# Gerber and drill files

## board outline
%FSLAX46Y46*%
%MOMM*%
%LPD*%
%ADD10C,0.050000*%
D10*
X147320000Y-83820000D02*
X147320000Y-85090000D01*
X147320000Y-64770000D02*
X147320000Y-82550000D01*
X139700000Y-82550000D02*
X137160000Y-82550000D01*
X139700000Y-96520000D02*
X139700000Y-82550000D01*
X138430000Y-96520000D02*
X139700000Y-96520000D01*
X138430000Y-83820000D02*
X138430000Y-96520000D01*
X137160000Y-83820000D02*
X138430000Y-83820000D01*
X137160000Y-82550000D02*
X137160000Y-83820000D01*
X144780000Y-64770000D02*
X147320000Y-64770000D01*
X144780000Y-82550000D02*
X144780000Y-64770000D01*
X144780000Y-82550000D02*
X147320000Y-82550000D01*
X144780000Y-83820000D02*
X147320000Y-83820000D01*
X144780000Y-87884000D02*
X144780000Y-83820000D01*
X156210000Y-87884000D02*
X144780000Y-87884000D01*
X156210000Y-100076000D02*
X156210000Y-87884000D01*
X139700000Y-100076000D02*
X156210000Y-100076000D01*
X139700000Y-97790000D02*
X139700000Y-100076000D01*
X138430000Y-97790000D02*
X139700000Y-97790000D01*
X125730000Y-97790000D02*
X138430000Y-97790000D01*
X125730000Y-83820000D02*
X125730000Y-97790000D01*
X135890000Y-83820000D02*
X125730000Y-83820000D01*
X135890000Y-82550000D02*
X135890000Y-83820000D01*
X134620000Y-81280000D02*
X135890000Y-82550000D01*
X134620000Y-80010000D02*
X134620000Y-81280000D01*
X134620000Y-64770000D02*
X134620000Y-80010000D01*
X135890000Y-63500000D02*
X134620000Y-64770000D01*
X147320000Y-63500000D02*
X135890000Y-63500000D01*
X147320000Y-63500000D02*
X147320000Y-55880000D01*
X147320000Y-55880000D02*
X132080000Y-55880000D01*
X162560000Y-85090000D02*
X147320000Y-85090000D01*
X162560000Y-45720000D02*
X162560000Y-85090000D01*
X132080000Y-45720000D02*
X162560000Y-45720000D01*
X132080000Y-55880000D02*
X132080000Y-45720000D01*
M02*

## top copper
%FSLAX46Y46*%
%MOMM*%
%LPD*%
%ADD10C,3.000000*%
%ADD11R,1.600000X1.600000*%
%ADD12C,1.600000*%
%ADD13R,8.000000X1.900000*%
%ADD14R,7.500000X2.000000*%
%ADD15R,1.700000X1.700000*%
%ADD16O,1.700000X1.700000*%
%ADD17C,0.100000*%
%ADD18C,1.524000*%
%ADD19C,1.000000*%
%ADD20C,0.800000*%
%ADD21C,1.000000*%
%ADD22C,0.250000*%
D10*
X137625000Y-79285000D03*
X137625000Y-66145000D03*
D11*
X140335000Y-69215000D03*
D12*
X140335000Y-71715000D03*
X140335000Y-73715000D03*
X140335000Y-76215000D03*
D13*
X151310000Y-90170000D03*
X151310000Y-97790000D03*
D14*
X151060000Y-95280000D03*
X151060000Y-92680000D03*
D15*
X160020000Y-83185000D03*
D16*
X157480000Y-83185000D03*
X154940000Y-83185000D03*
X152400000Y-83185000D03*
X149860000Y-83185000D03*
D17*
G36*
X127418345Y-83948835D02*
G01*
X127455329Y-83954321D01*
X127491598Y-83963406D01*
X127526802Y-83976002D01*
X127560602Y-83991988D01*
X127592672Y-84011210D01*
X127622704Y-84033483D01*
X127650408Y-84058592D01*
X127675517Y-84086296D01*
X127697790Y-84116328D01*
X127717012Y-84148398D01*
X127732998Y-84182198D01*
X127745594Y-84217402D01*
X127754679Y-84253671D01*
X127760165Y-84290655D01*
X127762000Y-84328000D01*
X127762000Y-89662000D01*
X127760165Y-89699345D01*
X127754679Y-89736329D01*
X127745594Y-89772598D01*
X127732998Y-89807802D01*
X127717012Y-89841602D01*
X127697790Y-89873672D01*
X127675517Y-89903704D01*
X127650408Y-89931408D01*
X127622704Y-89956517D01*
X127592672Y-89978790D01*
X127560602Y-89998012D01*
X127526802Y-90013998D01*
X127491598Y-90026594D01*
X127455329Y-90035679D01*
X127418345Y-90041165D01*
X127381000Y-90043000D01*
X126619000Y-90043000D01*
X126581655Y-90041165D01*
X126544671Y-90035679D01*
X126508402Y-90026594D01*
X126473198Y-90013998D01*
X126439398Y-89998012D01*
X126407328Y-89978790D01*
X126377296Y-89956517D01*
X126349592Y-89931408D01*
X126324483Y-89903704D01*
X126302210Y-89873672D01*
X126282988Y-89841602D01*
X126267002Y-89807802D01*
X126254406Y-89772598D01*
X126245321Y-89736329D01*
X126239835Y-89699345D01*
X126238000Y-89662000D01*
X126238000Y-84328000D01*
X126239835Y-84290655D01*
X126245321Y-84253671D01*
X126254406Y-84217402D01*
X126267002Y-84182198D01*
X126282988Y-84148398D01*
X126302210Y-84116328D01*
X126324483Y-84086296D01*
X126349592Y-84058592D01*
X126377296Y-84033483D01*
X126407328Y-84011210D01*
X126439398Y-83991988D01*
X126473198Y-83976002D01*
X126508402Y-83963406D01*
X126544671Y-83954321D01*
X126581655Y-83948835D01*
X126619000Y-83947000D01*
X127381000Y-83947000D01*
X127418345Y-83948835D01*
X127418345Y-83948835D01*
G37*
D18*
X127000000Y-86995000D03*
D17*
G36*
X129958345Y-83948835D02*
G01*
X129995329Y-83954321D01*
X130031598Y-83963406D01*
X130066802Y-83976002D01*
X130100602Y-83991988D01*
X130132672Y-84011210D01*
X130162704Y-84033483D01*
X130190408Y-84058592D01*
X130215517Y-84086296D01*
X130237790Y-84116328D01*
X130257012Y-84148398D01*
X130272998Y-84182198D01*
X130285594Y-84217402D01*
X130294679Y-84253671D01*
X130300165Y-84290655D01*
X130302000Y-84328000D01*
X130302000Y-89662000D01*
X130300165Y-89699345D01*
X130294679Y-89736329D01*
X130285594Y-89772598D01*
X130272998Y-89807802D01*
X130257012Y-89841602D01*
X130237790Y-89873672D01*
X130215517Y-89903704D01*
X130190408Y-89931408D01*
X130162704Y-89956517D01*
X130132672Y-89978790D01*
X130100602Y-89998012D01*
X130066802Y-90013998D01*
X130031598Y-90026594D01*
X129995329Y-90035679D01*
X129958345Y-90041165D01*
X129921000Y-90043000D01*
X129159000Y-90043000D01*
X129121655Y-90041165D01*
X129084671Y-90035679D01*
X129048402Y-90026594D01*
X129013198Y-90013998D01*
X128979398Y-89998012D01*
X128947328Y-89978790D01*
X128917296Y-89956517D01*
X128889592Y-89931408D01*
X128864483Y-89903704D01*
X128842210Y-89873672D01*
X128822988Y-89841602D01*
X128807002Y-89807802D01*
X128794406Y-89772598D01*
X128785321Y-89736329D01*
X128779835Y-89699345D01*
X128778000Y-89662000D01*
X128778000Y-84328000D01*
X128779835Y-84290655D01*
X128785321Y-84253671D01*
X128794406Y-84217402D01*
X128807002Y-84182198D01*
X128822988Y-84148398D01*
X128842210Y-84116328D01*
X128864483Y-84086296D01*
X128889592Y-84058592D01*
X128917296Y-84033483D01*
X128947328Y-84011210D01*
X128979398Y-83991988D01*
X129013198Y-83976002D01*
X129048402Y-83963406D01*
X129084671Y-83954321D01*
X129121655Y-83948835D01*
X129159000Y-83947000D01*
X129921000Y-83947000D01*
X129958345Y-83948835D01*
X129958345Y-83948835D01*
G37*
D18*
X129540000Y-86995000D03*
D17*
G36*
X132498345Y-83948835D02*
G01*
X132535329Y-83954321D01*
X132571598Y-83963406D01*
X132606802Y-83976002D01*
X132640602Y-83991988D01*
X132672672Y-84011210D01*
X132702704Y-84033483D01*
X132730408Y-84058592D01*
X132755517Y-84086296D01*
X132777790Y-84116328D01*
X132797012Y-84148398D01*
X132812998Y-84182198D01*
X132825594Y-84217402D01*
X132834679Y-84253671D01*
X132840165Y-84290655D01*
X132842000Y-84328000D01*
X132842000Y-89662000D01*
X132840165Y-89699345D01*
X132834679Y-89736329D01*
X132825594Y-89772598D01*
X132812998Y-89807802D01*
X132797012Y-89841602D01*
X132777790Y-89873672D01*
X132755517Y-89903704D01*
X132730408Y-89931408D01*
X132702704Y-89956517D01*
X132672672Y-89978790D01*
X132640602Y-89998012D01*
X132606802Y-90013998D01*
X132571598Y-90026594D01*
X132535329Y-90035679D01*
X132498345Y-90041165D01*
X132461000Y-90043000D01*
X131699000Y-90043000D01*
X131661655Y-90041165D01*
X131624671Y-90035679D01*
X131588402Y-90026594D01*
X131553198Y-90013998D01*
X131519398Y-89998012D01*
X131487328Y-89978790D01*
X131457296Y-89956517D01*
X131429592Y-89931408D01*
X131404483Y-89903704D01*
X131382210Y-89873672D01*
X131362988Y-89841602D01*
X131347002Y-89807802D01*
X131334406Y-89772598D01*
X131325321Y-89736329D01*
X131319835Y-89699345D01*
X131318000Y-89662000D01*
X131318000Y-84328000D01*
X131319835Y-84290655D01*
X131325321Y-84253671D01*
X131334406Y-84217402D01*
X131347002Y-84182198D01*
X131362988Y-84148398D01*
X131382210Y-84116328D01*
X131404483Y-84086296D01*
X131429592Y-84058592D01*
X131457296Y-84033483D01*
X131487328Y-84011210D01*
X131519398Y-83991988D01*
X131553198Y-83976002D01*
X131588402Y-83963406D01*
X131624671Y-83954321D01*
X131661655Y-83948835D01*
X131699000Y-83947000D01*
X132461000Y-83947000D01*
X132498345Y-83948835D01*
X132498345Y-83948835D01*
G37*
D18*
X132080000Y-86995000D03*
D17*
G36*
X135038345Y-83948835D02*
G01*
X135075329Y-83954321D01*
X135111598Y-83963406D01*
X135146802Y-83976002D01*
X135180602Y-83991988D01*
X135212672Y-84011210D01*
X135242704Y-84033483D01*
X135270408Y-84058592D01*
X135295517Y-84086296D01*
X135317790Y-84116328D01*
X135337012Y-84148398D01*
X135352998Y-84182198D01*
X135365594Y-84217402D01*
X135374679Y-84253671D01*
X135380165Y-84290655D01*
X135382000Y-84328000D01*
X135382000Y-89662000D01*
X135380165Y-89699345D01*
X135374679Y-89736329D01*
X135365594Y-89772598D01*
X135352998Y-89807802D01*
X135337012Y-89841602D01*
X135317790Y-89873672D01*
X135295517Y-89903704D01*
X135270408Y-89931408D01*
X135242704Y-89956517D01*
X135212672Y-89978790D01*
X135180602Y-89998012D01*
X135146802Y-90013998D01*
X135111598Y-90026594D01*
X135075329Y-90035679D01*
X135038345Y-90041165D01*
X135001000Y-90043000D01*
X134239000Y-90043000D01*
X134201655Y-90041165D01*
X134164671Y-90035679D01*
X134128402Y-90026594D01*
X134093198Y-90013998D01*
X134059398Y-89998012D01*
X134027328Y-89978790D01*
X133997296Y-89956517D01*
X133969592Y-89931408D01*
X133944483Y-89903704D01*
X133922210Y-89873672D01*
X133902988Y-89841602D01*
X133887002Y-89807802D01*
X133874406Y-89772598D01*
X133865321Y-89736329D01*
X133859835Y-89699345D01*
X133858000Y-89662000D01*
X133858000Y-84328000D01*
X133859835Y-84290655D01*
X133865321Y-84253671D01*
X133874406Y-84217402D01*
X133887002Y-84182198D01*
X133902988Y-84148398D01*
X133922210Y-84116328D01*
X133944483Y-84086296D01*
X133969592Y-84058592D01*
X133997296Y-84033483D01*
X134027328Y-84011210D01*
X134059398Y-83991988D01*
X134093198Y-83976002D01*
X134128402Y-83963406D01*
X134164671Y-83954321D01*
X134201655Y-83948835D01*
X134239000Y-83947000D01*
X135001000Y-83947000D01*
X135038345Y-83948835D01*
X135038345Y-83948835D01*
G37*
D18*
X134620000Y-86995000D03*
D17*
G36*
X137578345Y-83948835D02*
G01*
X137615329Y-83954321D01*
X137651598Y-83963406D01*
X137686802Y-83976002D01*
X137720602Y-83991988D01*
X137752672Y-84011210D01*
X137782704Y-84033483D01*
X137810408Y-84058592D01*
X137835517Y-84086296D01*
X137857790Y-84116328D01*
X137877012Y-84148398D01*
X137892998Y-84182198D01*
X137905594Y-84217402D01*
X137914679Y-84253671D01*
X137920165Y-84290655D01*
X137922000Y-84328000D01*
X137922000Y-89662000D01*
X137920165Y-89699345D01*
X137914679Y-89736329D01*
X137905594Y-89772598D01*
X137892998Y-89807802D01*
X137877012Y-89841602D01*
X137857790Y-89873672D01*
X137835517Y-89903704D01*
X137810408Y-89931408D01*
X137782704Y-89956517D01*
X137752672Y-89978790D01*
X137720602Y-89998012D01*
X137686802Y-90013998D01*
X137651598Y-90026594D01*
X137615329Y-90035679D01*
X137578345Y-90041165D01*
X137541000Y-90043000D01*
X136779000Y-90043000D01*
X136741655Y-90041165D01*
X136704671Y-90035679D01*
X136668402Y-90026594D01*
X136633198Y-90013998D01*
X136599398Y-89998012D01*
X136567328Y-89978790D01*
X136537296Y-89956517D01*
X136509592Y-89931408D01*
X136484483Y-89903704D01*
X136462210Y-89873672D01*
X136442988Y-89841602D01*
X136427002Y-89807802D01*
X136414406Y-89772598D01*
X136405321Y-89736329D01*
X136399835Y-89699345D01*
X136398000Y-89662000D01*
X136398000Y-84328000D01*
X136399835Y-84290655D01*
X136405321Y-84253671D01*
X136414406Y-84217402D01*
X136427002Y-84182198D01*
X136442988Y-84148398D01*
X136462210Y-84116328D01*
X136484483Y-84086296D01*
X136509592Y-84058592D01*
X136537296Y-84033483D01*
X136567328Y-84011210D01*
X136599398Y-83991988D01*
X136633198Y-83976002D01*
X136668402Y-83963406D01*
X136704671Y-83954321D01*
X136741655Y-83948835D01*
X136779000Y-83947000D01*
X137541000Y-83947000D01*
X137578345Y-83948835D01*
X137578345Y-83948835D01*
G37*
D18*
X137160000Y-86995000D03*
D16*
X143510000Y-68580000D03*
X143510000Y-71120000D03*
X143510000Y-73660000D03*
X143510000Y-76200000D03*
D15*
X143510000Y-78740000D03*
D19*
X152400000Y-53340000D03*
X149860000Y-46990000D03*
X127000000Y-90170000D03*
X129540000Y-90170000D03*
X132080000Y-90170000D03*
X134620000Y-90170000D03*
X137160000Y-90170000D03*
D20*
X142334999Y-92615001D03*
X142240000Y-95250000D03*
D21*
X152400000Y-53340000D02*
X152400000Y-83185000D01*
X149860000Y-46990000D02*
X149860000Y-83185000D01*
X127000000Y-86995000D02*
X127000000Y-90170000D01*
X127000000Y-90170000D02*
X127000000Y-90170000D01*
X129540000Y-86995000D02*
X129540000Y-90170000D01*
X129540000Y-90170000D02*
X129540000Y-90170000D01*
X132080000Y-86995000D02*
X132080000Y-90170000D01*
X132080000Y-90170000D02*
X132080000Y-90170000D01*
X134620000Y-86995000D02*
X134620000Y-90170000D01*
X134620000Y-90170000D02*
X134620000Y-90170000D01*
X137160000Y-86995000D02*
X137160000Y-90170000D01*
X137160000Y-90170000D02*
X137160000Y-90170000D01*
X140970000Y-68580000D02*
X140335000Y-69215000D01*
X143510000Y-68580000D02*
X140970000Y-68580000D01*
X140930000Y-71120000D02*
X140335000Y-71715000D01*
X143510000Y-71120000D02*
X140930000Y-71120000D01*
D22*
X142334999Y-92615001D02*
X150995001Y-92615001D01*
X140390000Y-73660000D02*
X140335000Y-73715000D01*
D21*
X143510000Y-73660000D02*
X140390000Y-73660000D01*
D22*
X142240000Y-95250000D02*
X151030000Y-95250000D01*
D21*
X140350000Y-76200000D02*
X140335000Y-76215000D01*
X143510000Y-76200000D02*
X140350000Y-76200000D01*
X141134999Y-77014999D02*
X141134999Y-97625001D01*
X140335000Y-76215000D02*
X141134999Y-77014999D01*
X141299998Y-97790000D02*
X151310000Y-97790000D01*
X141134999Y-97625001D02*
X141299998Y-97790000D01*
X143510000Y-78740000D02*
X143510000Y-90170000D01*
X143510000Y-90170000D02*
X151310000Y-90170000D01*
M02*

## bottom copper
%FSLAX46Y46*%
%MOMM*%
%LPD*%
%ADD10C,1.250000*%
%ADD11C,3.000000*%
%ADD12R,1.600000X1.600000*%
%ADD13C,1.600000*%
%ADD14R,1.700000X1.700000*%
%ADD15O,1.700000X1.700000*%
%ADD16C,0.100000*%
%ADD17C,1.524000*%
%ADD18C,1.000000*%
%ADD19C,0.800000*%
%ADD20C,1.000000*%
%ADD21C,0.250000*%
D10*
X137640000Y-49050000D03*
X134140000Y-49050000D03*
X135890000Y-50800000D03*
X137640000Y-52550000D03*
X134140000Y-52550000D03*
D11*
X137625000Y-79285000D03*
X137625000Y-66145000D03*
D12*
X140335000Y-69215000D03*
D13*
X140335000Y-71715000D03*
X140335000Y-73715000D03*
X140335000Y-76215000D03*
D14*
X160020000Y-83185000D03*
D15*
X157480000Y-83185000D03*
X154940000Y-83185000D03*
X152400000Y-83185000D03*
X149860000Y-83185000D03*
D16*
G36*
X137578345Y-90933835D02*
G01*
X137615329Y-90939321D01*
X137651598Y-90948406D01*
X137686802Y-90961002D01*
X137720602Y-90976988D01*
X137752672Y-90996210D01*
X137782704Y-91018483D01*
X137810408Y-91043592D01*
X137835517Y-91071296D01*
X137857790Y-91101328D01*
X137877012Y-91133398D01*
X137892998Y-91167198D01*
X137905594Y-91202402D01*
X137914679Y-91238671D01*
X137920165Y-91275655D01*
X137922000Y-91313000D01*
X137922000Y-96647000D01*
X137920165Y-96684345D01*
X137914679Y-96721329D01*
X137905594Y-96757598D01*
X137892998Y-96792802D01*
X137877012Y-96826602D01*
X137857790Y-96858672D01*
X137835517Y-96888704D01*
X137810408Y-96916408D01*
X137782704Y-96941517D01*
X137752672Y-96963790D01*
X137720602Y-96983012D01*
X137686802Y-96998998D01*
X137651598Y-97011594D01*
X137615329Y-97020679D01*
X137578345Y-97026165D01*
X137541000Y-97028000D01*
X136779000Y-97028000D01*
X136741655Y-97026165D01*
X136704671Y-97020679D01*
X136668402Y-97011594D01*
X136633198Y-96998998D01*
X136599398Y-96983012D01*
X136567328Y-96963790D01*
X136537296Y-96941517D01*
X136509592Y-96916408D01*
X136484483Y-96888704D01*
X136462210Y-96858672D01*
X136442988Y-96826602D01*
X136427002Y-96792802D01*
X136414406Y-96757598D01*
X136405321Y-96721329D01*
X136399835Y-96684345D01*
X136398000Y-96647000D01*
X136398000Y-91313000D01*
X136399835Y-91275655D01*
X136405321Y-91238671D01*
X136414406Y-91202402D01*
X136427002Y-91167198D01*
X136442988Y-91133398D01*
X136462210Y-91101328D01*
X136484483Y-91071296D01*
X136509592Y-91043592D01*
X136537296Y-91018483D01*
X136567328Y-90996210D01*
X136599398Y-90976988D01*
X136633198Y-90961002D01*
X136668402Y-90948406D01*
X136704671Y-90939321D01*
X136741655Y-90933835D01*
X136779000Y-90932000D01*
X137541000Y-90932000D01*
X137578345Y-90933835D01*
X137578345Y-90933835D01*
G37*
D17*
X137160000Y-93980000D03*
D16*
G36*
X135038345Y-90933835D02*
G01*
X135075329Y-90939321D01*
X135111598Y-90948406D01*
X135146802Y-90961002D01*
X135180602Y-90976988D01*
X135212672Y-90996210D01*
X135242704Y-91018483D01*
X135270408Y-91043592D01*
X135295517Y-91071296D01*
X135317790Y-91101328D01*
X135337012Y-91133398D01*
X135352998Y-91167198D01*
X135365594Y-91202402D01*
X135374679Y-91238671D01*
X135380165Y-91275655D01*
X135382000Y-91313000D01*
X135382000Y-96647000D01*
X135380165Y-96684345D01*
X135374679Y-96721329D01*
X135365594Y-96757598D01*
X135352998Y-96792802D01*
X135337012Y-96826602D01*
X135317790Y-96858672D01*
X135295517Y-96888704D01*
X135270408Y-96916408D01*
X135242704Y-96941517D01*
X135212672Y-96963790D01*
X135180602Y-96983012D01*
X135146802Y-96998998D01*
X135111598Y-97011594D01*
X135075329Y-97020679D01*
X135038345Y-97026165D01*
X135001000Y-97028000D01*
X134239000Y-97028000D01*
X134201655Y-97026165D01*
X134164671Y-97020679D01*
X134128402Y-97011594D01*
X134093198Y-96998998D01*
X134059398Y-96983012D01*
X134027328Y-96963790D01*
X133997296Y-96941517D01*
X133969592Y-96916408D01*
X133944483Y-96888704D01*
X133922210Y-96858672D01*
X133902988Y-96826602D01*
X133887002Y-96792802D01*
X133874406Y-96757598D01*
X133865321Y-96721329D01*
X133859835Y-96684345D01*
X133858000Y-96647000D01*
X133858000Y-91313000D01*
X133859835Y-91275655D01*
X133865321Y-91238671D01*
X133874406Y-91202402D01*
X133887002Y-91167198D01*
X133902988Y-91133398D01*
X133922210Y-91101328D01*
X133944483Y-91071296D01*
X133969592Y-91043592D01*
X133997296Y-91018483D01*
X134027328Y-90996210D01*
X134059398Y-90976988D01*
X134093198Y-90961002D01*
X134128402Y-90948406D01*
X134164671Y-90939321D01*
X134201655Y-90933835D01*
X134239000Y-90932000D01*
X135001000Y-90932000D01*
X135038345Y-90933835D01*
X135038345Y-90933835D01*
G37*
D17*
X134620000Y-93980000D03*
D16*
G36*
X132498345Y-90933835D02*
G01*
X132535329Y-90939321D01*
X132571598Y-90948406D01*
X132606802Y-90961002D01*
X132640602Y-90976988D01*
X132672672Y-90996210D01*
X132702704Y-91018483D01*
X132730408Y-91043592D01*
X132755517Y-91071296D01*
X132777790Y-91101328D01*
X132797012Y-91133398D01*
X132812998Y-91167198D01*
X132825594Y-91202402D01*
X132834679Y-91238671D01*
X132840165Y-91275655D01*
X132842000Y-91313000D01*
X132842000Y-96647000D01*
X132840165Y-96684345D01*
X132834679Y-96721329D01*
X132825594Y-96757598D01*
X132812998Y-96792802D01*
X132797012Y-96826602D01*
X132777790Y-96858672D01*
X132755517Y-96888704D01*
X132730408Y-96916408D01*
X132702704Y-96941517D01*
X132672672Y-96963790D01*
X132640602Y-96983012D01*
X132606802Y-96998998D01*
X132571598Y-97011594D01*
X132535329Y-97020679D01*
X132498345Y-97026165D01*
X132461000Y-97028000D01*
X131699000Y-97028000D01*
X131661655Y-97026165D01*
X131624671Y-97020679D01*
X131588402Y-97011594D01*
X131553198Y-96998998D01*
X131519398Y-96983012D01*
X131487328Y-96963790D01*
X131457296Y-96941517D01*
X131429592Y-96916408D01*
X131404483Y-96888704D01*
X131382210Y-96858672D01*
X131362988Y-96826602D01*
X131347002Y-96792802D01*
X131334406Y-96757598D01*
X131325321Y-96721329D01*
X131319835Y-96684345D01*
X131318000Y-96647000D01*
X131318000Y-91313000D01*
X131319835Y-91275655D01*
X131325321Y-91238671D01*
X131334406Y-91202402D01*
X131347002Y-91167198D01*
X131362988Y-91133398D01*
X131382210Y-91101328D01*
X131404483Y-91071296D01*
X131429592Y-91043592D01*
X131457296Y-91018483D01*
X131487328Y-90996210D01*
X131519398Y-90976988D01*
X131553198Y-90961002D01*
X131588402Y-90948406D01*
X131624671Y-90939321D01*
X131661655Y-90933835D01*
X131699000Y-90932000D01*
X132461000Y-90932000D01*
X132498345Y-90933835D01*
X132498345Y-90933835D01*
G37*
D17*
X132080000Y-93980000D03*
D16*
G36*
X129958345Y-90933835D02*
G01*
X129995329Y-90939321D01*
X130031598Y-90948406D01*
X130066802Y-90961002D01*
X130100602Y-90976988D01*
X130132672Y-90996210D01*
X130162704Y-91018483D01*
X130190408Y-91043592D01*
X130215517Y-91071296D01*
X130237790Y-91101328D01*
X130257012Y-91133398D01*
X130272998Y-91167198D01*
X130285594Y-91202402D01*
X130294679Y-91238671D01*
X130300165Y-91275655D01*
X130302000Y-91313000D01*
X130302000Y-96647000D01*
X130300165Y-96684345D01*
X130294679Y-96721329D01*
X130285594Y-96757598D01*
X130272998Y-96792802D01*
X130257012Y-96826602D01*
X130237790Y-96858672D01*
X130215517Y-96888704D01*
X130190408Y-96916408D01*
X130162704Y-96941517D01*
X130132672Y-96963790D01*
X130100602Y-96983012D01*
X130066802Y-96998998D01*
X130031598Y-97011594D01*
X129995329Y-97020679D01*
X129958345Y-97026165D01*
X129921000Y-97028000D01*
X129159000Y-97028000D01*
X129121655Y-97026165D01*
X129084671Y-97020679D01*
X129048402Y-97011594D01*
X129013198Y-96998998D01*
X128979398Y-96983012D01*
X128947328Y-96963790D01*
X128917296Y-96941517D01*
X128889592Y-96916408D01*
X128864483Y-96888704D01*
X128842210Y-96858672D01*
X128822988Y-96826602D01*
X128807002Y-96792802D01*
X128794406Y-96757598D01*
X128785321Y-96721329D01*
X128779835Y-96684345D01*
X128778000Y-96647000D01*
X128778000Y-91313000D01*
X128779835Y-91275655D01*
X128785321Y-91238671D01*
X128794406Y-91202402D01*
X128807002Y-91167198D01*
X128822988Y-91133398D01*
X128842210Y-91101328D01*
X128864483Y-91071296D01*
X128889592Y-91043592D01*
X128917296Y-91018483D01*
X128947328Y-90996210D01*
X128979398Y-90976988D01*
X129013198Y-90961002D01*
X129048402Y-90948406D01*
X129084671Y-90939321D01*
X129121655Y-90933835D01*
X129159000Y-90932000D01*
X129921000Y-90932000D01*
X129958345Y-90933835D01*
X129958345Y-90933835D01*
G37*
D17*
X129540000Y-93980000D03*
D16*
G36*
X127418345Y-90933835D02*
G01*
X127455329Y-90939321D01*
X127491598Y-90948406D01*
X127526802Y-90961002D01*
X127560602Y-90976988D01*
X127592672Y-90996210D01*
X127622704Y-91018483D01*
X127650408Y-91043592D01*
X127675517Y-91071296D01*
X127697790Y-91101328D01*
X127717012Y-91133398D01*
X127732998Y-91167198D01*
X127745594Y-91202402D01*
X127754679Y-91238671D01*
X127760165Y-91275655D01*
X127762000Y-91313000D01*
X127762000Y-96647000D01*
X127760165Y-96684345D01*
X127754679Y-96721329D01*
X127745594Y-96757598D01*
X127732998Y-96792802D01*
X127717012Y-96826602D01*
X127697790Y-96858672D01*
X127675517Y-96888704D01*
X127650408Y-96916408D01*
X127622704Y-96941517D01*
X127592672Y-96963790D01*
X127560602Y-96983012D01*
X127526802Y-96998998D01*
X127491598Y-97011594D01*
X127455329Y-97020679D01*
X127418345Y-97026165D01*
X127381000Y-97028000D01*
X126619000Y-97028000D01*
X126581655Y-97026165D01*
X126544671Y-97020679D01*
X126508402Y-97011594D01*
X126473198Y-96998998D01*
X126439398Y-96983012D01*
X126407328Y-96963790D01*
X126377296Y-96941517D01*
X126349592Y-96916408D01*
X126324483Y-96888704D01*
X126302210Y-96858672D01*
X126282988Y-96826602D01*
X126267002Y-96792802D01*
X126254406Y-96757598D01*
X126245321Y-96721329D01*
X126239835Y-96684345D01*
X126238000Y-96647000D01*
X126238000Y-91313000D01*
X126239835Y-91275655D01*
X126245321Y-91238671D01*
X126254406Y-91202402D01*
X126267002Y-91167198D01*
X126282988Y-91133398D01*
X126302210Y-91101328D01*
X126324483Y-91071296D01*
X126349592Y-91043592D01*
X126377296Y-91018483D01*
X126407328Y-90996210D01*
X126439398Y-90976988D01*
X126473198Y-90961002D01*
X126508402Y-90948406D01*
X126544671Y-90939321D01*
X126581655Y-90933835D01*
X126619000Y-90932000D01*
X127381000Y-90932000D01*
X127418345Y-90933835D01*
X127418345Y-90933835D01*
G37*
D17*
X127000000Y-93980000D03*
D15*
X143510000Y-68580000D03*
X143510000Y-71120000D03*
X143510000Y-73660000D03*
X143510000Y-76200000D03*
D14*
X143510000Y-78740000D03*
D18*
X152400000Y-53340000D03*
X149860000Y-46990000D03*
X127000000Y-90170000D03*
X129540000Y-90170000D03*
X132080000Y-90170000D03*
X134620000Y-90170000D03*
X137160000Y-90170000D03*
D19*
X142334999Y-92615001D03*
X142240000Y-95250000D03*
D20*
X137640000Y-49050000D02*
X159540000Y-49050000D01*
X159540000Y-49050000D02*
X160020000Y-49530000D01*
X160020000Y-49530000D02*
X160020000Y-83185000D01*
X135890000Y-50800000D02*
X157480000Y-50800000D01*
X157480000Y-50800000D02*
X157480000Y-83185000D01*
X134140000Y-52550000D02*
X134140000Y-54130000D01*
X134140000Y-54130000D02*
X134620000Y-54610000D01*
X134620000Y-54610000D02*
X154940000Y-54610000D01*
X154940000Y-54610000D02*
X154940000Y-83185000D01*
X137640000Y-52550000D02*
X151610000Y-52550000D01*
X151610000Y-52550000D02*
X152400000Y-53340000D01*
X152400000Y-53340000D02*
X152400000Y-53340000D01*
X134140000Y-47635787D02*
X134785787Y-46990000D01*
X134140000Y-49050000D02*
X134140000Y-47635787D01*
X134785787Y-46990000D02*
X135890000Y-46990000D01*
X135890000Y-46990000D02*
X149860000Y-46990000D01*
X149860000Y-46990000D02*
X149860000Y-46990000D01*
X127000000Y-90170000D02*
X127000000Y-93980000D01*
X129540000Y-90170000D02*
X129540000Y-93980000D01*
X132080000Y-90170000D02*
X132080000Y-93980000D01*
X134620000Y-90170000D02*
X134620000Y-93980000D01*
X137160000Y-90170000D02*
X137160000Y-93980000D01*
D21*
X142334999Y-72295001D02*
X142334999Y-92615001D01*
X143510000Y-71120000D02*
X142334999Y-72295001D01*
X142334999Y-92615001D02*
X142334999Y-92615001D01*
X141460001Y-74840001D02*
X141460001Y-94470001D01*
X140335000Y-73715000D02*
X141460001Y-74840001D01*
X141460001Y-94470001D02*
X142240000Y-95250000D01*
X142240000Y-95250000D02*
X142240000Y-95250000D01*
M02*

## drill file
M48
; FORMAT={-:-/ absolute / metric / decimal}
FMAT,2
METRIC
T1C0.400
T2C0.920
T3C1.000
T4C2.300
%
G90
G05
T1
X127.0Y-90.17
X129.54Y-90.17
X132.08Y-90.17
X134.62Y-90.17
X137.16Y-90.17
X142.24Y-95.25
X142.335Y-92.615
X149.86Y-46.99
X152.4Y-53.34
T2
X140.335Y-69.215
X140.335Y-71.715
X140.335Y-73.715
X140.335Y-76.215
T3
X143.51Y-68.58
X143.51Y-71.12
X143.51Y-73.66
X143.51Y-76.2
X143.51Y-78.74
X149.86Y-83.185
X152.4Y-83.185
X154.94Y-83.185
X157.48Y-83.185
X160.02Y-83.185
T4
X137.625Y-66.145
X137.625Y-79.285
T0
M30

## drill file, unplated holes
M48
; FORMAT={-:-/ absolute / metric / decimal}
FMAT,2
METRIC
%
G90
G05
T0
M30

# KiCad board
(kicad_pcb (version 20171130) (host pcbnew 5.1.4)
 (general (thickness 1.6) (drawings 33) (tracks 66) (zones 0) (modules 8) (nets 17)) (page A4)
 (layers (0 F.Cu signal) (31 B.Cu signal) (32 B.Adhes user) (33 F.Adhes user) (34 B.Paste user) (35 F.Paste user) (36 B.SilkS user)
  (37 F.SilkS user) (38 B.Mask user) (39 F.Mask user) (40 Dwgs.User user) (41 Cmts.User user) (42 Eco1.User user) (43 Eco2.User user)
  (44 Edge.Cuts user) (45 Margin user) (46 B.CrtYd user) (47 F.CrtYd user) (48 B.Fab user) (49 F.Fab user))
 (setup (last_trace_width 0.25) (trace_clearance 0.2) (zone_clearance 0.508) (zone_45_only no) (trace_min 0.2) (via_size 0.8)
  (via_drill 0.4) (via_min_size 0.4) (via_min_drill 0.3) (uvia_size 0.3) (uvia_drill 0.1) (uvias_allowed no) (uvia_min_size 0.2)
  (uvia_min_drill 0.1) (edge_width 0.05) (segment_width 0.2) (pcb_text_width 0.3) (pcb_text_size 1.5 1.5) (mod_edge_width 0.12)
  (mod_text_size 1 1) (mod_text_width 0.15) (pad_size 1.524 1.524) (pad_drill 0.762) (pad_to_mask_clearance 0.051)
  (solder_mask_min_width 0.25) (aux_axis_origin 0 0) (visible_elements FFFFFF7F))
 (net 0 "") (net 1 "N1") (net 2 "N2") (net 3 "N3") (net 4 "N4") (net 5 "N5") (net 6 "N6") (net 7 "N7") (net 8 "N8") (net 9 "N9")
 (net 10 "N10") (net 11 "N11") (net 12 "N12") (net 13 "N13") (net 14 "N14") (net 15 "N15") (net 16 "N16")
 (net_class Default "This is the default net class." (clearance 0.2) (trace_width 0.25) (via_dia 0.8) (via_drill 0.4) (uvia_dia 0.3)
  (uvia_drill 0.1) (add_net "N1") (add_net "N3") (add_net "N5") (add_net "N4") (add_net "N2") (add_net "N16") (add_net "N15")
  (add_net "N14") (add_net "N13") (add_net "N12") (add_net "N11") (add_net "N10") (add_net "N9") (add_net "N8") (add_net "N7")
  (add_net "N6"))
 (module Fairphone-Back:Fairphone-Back (layer F.Cu) (at 135.89 50.8)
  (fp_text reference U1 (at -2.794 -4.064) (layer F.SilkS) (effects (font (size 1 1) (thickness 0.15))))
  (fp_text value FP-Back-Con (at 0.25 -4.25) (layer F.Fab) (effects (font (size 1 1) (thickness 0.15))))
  (pad 2 connect circle (at 1.75 -1.75) (size 1.25 1.25) (layers B.Cu B.Mask) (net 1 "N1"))
  (pad 1 connect circle (at -1.75 -1.75) (size 1.25 1.25) (layers B.Cu B.Mask) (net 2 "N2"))
  (pad 3 connect circle (at 0 0) (size 1.25 1.25) (layers B.Cu B.Mask) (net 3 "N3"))
  (pad 5 connect circle (at 1.75 1.75) (size 1.25 1.25) (layers B.Cu B.Mask) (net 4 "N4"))
  (pad 4 connect circle (at -1.75 1.75) (size 1.25 1.25) (layers B.Cu B.Mask) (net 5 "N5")))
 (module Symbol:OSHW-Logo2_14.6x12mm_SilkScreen (layer F.Cu) (at 154.94 51.816)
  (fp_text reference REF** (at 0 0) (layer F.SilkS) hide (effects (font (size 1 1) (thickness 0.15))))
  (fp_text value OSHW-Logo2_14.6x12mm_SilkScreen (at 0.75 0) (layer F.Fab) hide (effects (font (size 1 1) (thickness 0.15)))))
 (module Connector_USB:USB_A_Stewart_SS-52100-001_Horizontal (layer F.Cu) (at 140.335 69.215 270)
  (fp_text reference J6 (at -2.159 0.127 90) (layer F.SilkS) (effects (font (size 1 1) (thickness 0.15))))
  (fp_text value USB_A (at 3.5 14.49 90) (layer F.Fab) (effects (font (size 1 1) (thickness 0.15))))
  (pad 5 thru_hole circle (at 10.07 2.71 270) (size 3 3) (drill 2.3) (layers *.Cu *.Mask) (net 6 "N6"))
  (pad 5 thru_hole circle (at -3.07 2.71 270) (size 3 3) (drill 2.3) (layers *.Cu *.Mask) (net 6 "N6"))
  (pad 1 thru_hole rect (at 0 0 270) (size 1.6 1.6) (drill 0.92) (layers *.Cu *.Mask) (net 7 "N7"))
  (pad 2 thru_hole circle (at 2.5 0 270) (size 1.6 1.6) (drill 0.92) (layers *.Cu *.Mask) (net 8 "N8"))
  (pad 3 thru_hole circle (at 4.5 0 270) (size 1.6 1.6) (drill 0.92) (layers *.Cu *.Mask) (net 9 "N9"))
  (pad 4 thru_hole circle (at 7 0 270) (size 1.6 1.6) (drill 0.92) (layers *.Cu *.Mask) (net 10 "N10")))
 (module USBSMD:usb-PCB (layer F.Cu) (at 156.21 93.98 90)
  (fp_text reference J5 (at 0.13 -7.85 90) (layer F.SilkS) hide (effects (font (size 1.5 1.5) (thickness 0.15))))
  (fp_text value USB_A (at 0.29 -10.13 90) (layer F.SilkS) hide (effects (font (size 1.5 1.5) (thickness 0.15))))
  (pad 1 connect rect (at 3.81 -4.9 90) (size 1.9 8) (layers F.Cu F.Mask) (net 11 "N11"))
  (pad 4 connect rect (at -3.81 -4.9 90) (size 1.9 8) (layers F.Cu F.Mask) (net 10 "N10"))
  (pad 3 connect rect (at -1.3 -5.15 90) (size 2 7.5) (layers F.Cu F.Mask) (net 9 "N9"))
  (pad 2 connect rect (at 1.3 -5.15 90) (size 2 7.5) (layers F.Cu F.Mask) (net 8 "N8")))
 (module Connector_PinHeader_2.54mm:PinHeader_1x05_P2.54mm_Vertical (layer F.Cu) (at 160.02 83.185 270)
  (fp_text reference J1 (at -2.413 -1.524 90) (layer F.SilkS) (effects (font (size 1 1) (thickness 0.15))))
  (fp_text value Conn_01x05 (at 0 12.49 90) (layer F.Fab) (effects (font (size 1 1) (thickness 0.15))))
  (pad 1 thru_hole rect (at 0 0 270) (size 1.7 1.7) (drill 1) (layers *.Cu *.Mask) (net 1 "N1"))
  (pad 2 thru_hole oval (at 0 2.54 270) (size 1.7 1.7) (drill 1) (layers *.Cu *.Mask) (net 3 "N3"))
  (pad 3 thru_hole oval (at 0 5.08 270) (size 1.7 1.7) (drill 1) (layers *.Cu *.Mask) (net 5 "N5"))
  (pad 4 thru_hole oval (at 0 7.62 270) (size 1.7 1.7) (drill 1) (layers *.Cu *.Mask) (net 4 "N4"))
  (pad 5 thru_hole oval (at 0 10.16 270) (size 1.7 1.7) (drill 1) (layers *.Cu *.Mask) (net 2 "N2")))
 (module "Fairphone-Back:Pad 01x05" (layer B.Cu) (at 132.08 93.98)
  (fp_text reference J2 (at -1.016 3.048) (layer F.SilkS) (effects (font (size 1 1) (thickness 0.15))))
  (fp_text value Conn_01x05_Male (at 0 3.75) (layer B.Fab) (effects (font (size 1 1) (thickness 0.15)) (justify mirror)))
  (pad 5 smd roundrect (at 5.08 0) (size 1.524 6.096) (layers B.Cu B.Paste B.Mask) (roundrect_rratio 0.25) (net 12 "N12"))
  (pad 4 smd roundrect (at 2.54 0) (size 1.524 6.096) (layers B.Cu B.Paste B.Mask) (roundrect_rratio 0.25) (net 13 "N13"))
  (pad 3 smd roundrect (at 0 0) (size 1.524 6.096) (layers B.Cu B.Paste B.Mask) (roundrect_rratio 0.25) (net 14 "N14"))
  (pad 2 smd roundrect (at -2.54 0) (size 1.524 6.096) (layers B.Cu B.Paste B.Mask) (roundrect_rratio 0.25) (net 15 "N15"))
  (pad 1 smd roundrect (at -5.08 0) (size 1.524 6.096) (layers B.Cu B.Paste B.Mask) (roundrect_rratio 0.25) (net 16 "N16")))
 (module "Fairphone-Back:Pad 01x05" (layer F.Cu) (at 132.08 86.995)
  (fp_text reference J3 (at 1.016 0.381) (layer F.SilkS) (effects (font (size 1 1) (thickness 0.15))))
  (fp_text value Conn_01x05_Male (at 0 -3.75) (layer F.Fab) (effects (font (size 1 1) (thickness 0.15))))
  (pad 1 smd roundrect (at -5.08 0) (size 1.524 6.096) (layers F.Cu F.Paste F.Mask) (roundrect_rratio 0.25) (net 16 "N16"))
  (pad 2 smd roundrect (at -2.54 0) (size 1.524 6.096) (layers F.Cu F.Paste F.Mask) (roundrect_rratio 0.25) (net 15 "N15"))
  (pad 3 smd roundrect (at 0 0) (size 1.524 6.096) (layers F.Cu F.Paste F.Mask) (roundrect_rratio 0.25) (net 14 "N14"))
  (pad 4 smd roundrect (at 2.54 0) (size 1.524 6.096) (layers F.Cu F.Paste F.Mask) (roundrect_rratio 0.25) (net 13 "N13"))
  (pad 5 smd roundrect (at 5.08 0) (size 1.524 6.096) (layers F.Cu F.Paste F.Mask) (roundrect_rratio 0.25) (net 12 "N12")))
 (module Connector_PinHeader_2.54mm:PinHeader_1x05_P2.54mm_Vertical (layer F.Cu) (at 143.51 78.74 180)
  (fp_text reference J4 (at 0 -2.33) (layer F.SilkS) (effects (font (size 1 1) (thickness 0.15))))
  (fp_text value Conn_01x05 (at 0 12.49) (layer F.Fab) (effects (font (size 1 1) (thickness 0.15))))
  (pad 5 thru_hole oval (at 0 10.16 180) (size 1.7 1.7) (drill 1) (layers *.Cu *.Mask) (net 7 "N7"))
  (pad 4 thru_hole oval (at 0 7.62 180) (size 1.7 1.7) (drill 1) (layers *.Cu *.Mask) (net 8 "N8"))
  (pad 3 thru_hole oval (at 0 5.08 180) (size 1.7 1.7) (drill 1) (layers *.Cu *.Mask) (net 9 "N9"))
  (pad 2 thru_hole oval (at 0 2.54 180) (size 1.7 1.7) (drill 1) (layers *.Cu *.Mask) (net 10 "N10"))
  (pad 1 thru_hole rect (at 0 0 180) (size 1.7 1.7) (drill 1) (layers *.Cu *.Mask) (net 11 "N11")))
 (gr_line (start 147.32 83.82) (end 147.32 85.09) (layer Edge.Cuts) (width 0.05))
 (gr_line (start 147.32 64.77) (end 147.32 82.55) (layer Edge.Cuts) (width 0.05))
 (gr_line (start 139.7 82.55) (end 137.16 82.55) (layer Edge.Cuts) (width 0.05))
 (gr_line (start 139.7 96.52) (end 139.7 82.55) (layer Edge.Cuts) (width 0.05))
 (gr_line (start 138.43 96.52) (end 139.7 96.52) (layer Edge.Cuts) (width 0.05))
 (gr_line (start 138.43 83.82) (end 138.43 96.52) (layer Edge.Cuts) (width 0.05))
 (gr_line (start 137.16 83.82) (end 138.43 83.82) (layer Edge.Cuts) (width 0.05))
 (gr_line (start 137.16 82.55) (end 137.16 83.82) (layer Edge.Cuts) (width 0.05))
 (gr_line (start 144.78 64.77) (end 147.32 64.77) (layer Edge.Cuts) (width 0.05))
 (gr_line (start 144.78 82.55) (end 144.78 64.77) (layer Edge.Cuts) (width 0.05))
 (gr_line (start 144.78 82.55) (end 147.32 82.55) (layer Edge.Cuts) (width 0.05))
 (gr_line (start 144.78 83.82) (end 147.32 83.82) (layer Edge.Cuts) (width 0.05))
 (gr_line (start 144.78 87.884) (end 144.78 83.82) (layer Edge.Cuts) (width 0.05))
 (gr_line (start 156.21 87.884) (end 144.78 87.884) (layer Edge.Cuts) (width 0.05))
 (gr_line (start 156.21 100.076) (end 156.21 87.884) (layer Edge.Cuts) (width 0.05))
 (gr_line (start 139.7 100.076) (end 156.21 100.076) (layer Edge.Cuts) (width 0.05))
 (gr_line (start 139.7 97.79) (end 139.7 100.076) (layer Edge.Cuts) (width 0.05))
 (gr_line (start 138.43 97.79) (end 139.7 97.79) (layer Edge.Cuts) (width 0.05))
 (gr_line (start 125.73 97.79) (end 138.43 97.79) (layer Edge.Cuts) (width 0.05))
 (gr_line (start 125.73 83.82) (end 125.73 97.79) (layer Edge.Cuts) (width 0.05))
 (gr_line (start 135.89 83.82) (end 125.73 83.82) (layer Edge.Cuts) (width 0.05))
 (gr_line (start 135.89 82.55) (end 135.89 83.82) (layer Edge.Cuts) (width 0.05))
 (gr_line (start 134.62 81.28) (end 135.89 82.55) (layer Edge.Cuts) (width 0.05))
 (gr_line (start 134.62 80.01) (end 134.62 81.28) (layer Edge.Cuts) (width 0.05))
 (gr_line (start 134.62 64.77) (end 134.62 80.01) (layer Edge.Cuts) (width 0.05))
 (gr_line (start 135.89 63.5) (end 134.62 64.77) (layer Edge.Cuts) (width 0.05))
 (gr_line (start 147.32 63.5) (end 135.89 63.5) (layer Edge.Cuts) (width 0.05))
 (gr_line (start 147.32 63.5) (end 147.32 55.88) (layer Edge.Cuts) (width 0.05))
 (gr_line (start 147.32 55.88) (end 132.08 55.88) (layer Edge.Cuts) (width 0.05))
 (gr_line (start 162.56 85.09) (end 147.32 85.09) (layer Edge.Cuts) (width 0.05))
 (gr_line (start 162.56 45.72) (end 162.56 85.09) (layer Edge.Cuts) (width 0.05))
 (gr_line (start 132.08 45.72) (end 162.56 45.72) (layer Edge.Cuts) (width 0.05))
 (gr_line (start 132.08 55.88) (end 132.08 45.72) (layer Edge.Cuts) (width 0.05))
 (segment (start 137.64 49.05) (end 159.54 49.05) (width 1) (layer B.Cu) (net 1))
 (segment (start 159.54 49.05) (end 160.02 49.53) (width 1) (layer B.Cu) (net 1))
 (segment (start 160.02 49.53) (end 160.02 83.185) (width 1) (layer B.Cu) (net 1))
 (segment (start 135.89 50.8) (end 157.48 50.8) (width 1) (layer B.Cu) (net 3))
 (segment (start 157.48 50.8) (end 157.48 83.185) (width 1) (layer B.Cu) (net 3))
 (segment (start 134.14 52.55) (end 134.14 54.13) (width 1) (layer B.Cu) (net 5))
 (segment (start 134.14 54.13) (end 134.62 54.61) (width 1) (layer B.Cu) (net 5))
 (segment (start 134.62 54.61) (end 154.94 54.61) (width 1) (layer B.Cu) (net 5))
 (segment (start 154.94 54.61) (end 154.94 83.185) (width 1) (layer B.Cu) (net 5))
 (segment (start 137.64 52.55) (end 151.61 52.55) (width 1) (layer B.Cu) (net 4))
 (segment (start 151.61 52.55) (end 152.4 53.34) (width 1) (layer B.Cu) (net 4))
 (segment (start 152.4 53.34) (end 152.4 53.34) (width 1) (layer B.Cu) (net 4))
 (via (at 152.4 53.34) (size 1) (drill 0.4) (layers F.Cu B.Cu) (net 4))
 (segment (start 152.4 53.34) (end 152.4 83.185) (width 1) (layer F.Cu) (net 4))
 (segment (start 134.14 47.635787) (end 134.785787 46.99) (width 1) (layer B.Cu) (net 2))
 (segment (start 134.14 49.05) (end 134.14 47.635787) (width 1) (layer B.Cu) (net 2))
 (segment (start 134.785787 46.99) (end 135.89 46.99) (width 1) (layer B.Cu) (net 2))
 (segment (start 135.89 46.99) (end 149.86 46.99) (width 1) (layer B.Cu) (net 2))
 (segment (start 149.86 46.99) (end 149.86 46.99) (width 1) (layer B.Cu) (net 2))
 (via (at 149.86 46.99) (size 1) (drill 0.4) (layers F.Cu B.Cu) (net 2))
 (segment (start 149.86 46.99) (end 149.86 83.185) (width 1) (layer F.Cu) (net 2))
 (segment (start 127 86.995) (end 127 90.17) (width 1) (layer F.Cu) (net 16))
 (segment (start 127 90.17) (end 127 90.17) (width 1) (layer F.Cu) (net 16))
 (via (at 127 90.17) (size 1) (drill 0.4) (layers F.Cu B.Cu) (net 16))
 (segment (start 127 90.17) (end 127 93.98) (width 1) (layer B.Cu) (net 16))
 (segment (start 129.54 86.995) (end 129.54 90.17) (width 1) (layer F.Cu) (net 15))
 (segment (start 129.54 90.17) (end 129.54 90.17) (width 1) (layer F.Cu) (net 15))
 (via (at 129.54 90.17) (size 1) (drill 0.4) (layers F.Cu B.Cu) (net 15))
 (segment (start 129.54 90.17) (end 129.54 93.98) (width 1) (layer B.Cu) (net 15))
 (segment (start 132.08 86.995) (end 132.08 90.17) (width 1) (layer F.Cu) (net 14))
 (segment (start 132.08 90.17) (end 132.08 90.17) (width 1) (layer F.Cu) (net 14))
 (via (at 132.08 90.17) (size 1) (drill 0.4) (layers F.Cu B.Cu) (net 14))
 (segment (start 132.08 90.17) (end 132.08 93.98) (width 1) (layer B.Cu) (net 14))
 (segment (start 134.62 86.995) (end 134.62 90.17) (width 1) (layer F.Cu) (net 13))
 (segment (start 134.62 90.17) (end 134.62 90.17) (width 1) (layer F.Cu) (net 13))
 (via (at 134.62 90.17) (size 1) (drill 0.4) (layers F.Cu B.Cu) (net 13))
 (segment (start 134.62 90.17) (end 134.62 93.98) (width 1) (layer B.Cu) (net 13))
 (segment (start 137.16 86.995) (end 137.16 90.17) (width 1) (layer F.Cu) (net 12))
 (segment (start 137.16 90.17) (end 137.16 90.17) (width 1) (layer F.Cu) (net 12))
 (via (at 137.16 90.17) (size 1) (drill 0.4) (layers F.Cu B.Cu) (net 12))
 (segment (start 137.16 90.17) (end 137.16 93.98) (width 1) (layer B.Cu) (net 12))
 (segment (start 140.97 68.58) (end 140.335 69.215) (width 1) (layer F.Cu) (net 7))
 (segment (start 143.51 68.58) (end 140.97 68.58) (width 1) (layer F.Cu) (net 7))
 (segment (start 140.93 71.12) (end 140.335 71.715) (width 1) (layer F.Cu) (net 8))
 (segment (start 143.51 71.12) (end 140.93 71.12) (width 1) (layer F.Cu) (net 8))
 (segment (start 142.334999 72.295001) (end 142.334999 92.615001) (width 0.25) (layer B.Cu) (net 8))
 (segment (start 143.51 71.12) (end 142.334999 72.295001) (width 0.25) (layer B.Cu) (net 8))
 (segment (start 142.334999 92.615001) (end 142.334999 92.615001) (width 0.25) (layer B.Cu) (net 8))
 (via (at 142.334999 92.615001) (size 0.8) (drill 0.4) (layers F.Cu B.Cu) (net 8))
 (segment (start 142.334999 92.615001) (end 150.995001 92.615001) (width 0.25) (layer F.Cu) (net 8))
 (segment (start 140.39 73.66) (end 140.335 73.715) (width 0.25) (layer F.Cu) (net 9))
 (segment (start 143.51 73.66) (end 140.39 73.66) (width 1) (layer F.Cu) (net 9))
 (segment (start 141.460001 74.840001) (end 141.460001 94.470001) (width 0.25) (layer B.Cu) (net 9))
 (segment (start 140.335 73.715) (end 141.460001 74.840001) (width 0.25) (layer B.Cu) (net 9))
 (segment (start 141.460001 94.470001) (end 142.24 95.25) (width 0.25) (layer B.Cu) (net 9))
 (segment (start 142.24 95.25) (end 142.24 95.25) (width 0.25) (layer B.Cu) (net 9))
 (via (at 142.24 95.25) (size 0.8) (drill 0.4) (layers F.Cu B.Cu) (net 9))
 (segment (start 142.24 95.25) (end 151.03 95.25) (width 0.25) (layer F.Cu) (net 9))
 (segment (start 140.35 76.2) (end 140.335 76.215) (width 1) (layer F.Cu) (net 10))
 (segment (start 143.51 76.2) (end 140.35 76.2) (width 1) (layer F.Cu) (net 10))
 (segment (start 141.134999 77.014999) (end 141.134999 97.625001) (width 1) (layer F.Cu) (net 10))
 (segment (start 140.335 76.215) (end 141.134999 77.014999) (width 1) (layer F.Cu) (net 10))
 (segment (start 141.299998 97.79) (end 151.31 97.79) (width 1) (layer F.Cu) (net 10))
 (segment (start 141.134999 97.625001) (end 141.299998 97.79) (width 1) (layer F.Cu) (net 10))
 (segment (start 143.51 78.74) (end 143.51 90.17) (width 1) (layer F.Cu) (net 11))
 (segment (start 143.51 90.17) (end 151.31 90.17) (width 1) (layer F.Cu) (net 11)))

